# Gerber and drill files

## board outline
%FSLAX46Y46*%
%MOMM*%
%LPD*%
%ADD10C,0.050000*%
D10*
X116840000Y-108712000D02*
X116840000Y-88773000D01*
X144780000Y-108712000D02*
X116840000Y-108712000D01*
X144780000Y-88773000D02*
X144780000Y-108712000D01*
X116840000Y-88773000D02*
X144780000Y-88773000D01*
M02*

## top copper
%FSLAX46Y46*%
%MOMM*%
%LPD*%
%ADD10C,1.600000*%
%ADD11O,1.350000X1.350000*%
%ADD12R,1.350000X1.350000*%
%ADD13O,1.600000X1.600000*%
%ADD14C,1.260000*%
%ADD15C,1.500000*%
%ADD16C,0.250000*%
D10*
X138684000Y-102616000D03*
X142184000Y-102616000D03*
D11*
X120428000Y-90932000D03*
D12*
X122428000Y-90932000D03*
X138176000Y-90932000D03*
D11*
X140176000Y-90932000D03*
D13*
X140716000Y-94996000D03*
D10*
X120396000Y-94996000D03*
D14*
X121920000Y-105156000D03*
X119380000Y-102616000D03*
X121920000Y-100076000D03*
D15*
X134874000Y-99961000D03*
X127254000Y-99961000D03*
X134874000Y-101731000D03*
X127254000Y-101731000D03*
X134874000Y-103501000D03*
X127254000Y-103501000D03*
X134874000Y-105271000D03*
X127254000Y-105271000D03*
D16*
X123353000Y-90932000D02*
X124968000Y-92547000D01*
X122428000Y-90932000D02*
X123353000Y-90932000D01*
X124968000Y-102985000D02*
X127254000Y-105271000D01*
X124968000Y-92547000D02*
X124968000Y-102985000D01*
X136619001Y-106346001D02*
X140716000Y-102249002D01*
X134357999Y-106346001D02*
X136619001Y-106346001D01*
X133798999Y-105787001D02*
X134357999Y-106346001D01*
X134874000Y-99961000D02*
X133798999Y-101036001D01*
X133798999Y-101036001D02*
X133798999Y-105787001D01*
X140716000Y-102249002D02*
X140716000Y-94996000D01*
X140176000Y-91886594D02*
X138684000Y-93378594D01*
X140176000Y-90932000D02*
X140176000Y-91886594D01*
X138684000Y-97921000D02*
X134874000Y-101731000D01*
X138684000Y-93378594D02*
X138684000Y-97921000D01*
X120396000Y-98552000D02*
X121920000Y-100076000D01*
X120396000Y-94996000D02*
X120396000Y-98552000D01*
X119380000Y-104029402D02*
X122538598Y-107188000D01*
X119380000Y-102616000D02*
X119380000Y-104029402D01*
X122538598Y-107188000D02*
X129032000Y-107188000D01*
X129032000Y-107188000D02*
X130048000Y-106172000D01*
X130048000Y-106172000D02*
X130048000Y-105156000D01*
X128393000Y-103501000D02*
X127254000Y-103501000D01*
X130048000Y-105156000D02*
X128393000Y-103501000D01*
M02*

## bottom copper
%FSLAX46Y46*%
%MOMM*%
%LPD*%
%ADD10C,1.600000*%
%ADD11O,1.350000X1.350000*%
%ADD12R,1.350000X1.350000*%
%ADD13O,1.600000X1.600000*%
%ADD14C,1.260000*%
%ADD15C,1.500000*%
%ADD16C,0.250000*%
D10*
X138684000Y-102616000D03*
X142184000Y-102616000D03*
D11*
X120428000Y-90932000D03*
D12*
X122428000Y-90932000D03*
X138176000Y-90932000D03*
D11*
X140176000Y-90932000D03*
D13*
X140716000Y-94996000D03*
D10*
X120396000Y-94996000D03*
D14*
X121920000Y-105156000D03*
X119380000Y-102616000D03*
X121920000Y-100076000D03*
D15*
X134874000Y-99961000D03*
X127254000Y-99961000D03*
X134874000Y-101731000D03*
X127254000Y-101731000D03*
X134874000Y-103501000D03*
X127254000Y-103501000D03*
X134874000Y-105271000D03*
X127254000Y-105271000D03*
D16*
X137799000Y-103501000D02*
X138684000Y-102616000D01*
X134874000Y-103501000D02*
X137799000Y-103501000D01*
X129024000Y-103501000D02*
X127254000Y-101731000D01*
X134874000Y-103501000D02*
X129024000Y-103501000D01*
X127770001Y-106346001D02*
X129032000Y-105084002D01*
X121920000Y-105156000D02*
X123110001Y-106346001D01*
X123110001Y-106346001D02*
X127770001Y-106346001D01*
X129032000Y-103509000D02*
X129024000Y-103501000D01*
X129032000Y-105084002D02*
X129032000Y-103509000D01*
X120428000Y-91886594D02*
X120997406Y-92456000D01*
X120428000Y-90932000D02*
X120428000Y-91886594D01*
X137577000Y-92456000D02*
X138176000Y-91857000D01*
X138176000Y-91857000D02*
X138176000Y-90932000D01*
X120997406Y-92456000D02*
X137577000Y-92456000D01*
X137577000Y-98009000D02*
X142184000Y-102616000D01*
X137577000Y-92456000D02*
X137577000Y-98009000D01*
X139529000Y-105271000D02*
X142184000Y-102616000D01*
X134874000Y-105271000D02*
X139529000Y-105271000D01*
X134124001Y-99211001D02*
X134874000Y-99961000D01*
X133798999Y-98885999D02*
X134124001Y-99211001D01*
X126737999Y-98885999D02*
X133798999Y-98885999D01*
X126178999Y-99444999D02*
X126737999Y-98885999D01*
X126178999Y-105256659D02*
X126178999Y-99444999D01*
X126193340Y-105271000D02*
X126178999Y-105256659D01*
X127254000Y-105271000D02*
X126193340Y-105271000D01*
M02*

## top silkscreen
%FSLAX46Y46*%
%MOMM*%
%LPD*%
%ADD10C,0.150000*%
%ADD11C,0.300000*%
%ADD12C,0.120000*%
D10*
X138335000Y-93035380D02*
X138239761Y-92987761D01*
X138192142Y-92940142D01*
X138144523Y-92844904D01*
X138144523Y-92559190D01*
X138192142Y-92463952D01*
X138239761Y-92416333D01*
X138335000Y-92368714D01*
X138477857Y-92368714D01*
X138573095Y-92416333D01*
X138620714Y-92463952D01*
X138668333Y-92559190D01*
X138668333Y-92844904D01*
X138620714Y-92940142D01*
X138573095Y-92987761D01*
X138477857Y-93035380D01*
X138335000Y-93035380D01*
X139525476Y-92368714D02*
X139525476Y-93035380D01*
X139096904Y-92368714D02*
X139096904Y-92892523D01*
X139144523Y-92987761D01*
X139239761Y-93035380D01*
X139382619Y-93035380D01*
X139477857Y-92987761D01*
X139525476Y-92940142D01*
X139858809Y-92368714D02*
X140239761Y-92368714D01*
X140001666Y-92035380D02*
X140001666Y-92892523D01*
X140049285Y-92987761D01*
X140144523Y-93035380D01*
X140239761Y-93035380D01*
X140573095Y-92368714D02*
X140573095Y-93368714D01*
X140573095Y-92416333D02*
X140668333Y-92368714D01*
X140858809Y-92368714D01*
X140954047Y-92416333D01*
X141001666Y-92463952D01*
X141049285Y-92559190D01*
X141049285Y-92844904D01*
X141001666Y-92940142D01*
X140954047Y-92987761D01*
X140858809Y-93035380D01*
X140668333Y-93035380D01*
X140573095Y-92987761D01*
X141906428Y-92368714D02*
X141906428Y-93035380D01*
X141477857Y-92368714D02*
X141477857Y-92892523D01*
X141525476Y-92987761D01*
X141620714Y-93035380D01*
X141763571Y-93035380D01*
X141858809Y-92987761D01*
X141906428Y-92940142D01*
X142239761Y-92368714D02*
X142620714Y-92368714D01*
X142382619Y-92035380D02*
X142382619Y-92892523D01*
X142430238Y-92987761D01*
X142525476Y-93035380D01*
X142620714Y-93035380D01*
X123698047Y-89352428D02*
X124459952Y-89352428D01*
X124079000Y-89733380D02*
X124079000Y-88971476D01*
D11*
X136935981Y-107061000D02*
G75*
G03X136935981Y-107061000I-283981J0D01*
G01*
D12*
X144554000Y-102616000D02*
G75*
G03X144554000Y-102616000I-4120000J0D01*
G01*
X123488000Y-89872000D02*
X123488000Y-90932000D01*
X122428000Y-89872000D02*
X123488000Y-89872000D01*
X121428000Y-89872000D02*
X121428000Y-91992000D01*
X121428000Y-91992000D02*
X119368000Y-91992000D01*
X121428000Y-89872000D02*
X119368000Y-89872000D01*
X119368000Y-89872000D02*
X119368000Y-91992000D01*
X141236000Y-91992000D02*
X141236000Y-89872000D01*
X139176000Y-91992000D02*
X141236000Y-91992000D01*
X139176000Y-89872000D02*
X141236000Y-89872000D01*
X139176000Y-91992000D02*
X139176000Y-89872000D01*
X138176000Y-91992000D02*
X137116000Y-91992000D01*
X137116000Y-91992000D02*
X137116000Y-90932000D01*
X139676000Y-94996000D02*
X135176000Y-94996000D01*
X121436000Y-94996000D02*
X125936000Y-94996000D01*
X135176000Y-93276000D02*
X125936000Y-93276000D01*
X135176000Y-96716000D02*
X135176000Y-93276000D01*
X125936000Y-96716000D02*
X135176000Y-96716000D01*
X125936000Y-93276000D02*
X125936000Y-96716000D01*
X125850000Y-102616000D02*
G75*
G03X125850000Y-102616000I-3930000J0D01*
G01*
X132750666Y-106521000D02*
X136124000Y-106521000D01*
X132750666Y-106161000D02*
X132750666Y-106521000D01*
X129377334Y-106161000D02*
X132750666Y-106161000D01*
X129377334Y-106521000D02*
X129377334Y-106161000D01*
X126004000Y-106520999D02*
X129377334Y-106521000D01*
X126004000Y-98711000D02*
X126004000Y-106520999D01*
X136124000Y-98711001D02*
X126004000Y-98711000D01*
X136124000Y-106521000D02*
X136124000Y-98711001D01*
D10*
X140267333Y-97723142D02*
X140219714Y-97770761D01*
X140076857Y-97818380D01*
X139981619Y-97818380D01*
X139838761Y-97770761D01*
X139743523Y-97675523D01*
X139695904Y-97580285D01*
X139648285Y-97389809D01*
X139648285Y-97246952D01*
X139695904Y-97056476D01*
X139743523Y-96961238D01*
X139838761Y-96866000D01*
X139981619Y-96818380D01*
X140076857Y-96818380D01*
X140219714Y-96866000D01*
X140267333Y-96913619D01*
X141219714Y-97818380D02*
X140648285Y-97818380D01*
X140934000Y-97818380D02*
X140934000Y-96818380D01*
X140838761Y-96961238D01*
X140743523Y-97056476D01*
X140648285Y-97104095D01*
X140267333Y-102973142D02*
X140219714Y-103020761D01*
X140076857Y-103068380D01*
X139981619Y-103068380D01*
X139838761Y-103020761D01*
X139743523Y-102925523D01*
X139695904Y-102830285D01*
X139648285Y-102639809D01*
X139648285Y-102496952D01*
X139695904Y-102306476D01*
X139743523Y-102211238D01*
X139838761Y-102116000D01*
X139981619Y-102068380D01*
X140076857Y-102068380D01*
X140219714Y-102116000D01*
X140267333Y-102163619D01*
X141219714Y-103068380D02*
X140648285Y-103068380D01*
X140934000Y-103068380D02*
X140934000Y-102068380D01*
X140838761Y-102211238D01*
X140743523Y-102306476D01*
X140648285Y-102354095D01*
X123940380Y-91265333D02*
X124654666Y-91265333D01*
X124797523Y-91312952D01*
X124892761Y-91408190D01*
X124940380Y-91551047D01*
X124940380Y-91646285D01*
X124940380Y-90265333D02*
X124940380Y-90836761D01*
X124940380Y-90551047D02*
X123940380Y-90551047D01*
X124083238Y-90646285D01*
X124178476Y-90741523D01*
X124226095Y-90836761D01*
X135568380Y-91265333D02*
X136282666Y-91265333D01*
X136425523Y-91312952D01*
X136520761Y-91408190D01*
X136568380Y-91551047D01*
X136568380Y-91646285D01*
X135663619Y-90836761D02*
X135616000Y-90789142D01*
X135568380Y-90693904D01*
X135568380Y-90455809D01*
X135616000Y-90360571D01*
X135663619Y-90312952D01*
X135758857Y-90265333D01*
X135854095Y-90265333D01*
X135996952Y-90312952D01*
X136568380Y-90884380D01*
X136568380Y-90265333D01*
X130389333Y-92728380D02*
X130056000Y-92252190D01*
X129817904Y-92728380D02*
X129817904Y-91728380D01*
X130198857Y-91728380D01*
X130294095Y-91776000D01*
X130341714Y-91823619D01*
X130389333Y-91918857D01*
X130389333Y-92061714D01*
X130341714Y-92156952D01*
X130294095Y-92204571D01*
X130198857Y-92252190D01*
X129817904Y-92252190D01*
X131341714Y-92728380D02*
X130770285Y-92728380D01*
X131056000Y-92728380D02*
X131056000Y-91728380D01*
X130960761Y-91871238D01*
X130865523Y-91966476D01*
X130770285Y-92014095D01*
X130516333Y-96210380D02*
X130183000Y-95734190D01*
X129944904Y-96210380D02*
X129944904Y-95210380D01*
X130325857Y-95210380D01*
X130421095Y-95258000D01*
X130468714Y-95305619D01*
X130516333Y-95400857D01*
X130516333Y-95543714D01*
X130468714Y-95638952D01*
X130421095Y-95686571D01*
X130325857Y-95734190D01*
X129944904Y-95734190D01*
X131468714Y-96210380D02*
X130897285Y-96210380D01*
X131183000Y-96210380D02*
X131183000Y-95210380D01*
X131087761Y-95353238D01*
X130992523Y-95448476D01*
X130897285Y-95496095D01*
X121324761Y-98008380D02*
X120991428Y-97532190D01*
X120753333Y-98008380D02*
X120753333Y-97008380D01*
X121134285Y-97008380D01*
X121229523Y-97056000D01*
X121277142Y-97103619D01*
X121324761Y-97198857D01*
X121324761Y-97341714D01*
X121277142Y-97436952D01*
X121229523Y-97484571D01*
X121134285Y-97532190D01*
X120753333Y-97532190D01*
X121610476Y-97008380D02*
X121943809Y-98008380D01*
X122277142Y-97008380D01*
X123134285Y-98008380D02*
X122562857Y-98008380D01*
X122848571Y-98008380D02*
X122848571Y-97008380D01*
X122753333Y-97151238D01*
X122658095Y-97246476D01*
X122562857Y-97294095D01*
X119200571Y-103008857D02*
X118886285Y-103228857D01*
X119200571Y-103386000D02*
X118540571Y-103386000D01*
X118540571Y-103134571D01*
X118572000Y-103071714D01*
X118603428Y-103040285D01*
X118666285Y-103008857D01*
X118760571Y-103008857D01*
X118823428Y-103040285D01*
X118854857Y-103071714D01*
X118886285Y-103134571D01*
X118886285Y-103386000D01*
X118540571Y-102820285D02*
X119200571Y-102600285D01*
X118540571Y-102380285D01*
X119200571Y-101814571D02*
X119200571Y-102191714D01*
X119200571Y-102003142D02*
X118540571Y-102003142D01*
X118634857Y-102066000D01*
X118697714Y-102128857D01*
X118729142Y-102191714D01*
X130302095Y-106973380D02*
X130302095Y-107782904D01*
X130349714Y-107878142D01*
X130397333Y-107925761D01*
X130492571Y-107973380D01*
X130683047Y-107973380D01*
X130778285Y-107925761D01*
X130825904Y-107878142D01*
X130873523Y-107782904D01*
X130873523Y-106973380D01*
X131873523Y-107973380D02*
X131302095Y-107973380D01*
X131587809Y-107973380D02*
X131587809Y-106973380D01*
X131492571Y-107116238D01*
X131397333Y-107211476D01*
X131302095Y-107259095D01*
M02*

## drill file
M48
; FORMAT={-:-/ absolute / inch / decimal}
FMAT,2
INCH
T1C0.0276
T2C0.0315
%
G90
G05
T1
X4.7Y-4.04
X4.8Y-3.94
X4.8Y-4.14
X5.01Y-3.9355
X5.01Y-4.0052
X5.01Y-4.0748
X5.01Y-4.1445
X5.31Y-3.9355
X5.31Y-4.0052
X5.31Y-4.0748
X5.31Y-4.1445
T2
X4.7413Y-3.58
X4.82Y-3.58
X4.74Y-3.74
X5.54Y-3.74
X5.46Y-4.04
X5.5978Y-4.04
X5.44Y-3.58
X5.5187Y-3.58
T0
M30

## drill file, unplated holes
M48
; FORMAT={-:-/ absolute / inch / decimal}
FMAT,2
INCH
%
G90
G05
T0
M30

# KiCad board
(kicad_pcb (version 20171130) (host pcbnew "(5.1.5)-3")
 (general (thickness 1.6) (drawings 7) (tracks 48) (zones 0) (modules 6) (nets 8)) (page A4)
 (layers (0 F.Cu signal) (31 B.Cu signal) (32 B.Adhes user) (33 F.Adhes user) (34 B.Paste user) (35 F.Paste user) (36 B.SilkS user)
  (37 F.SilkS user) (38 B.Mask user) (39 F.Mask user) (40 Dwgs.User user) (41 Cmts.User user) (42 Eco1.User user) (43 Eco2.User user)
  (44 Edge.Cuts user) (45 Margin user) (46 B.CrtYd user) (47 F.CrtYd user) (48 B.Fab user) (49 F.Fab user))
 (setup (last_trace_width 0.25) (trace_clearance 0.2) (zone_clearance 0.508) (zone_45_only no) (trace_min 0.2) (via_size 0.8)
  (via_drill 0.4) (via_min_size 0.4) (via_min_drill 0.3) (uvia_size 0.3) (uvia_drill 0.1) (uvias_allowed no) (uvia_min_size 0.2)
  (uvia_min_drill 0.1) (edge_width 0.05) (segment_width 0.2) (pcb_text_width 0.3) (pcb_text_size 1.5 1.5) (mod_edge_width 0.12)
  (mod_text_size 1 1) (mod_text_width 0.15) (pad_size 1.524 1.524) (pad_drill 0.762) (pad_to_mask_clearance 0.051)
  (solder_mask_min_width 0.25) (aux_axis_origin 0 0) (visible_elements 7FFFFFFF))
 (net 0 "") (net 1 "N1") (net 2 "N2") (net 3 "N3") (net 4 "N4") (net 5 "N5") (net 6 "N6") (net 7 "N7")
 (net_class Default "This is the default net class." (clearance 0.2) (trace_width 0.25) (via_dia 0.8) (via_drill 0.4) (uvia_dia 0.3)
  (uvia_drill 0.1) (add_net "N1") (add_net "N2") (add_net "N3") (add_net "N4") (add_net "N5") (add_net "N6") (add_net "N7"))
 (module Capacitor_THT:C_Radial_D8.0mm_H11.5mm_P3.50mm (layer F.Cu) (at 138.684 102.616)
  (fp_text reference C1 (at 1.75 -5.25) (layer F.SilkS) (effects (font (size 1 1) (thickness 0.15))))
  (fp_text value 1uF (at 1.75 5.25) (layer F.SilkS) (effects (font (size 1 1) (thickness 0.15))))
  (fp_circle (center 1.75 0) (end 5.87 0) (layer F.SilkS) (width 0.12))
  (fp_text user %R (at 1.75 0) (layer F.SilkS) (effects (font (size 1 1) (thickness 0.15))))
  (pad 1 thru_hole circle (at 0 0) (size 1.6 1.6) (drill 0.8) (layers *.Cu *.Mask) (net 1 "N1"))
  (pad 2 thru_hole circle (at 3.5 0) (size 1.6 1.6) (drill 0.8) (layers *.Cu *.Mask) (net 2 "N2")))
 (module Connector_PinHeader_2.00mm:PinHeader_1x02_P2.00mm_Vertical (layer F.Cu) (at 122.428 90.932 270)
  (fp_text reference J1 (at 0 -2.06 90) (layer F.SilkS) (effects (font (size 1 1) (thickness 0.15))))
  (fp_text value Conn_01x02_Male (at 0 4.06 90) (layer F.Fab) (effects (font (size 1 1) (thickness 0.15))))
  (fp_line (start -1.06 -1.06) (end 0 -1.06) (layer F.SilkS) (width 0.12))
  (fp_line (start -1.06 0) (end -1.06 -1.06) (layer F.SilkS) (width 0.12))
  (fp_line (start -1.06 1) (end 1.06 1) (layer F.SilkS) (width 0.12))
  (fp_line (start 1.06 1) (end 1.06 3.06) (layer F.SilkS) (width 0.12))
  (fp_line (start -1.06 1) (end -1.06 3.06) (layer F.SilkS) (width 0.12))
  (fp_line (start -1.06 3.06) (end 1.06 3.06) (layer F.SilkS) (width 0.12))
  (pad 2 thru_hole oval (at 0 2 270) (size 1.35 1.35) (drill 0.8) (layers *.Cu *.Mask) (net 2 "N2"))
  (pad 1 thru_hole rect (at 0 0 270) (size 1.35 1.35) (drill 0.8) (layers *.Cu *.Mask) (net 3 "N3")))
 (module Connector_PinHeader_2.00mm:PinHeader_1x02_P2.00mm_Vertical (layer F.Cu) (at 138.176 90.932 90)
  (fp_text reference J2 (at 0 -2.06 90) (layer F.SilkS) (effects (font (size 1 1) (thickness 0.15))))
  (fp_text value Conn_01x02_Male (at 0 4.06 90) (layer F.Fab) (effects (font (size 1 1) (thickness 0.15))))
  (fp_line (start -1.06 3.06) (end 1.06 3.06) (layer F.SilkS) (width 0.12))
  (fp_line (start -1.06 1) (end -1.06 3.06) (layer F.SilkS) (width 0.12))
  (fp_line (start 1.06 1) (end 1.06 3.06) (layer F.SilkS) (width 0.12))
  (fp_line (start -1.06 1) (end 1.06 1) (layer F.SilkS) (width 0.12))
  (fp_line (start -1.06 0) (end -1.06 -1.06) (layer F.SilkS) (width 0.12))
  (fp_line (start -1.06 -1.06) (end 0 -1.06) (layer F.SilkS) (width 0.12))
  (pad 1 thru_hole rect (at 0 0 90) (size 1.35 1.35) (drill 0.8) (layers *.Cu *.Mask) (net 2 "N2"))
  (pad 2 thru_hole oval (at 0 2 90) (size 1.35 1.35) (drill 0.8) (layers *.Cu *.Mask) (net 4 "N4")))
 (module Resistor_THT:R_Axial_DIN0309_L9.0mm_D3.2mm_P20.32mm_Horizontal (layer F.Cu) (at 120.396 94.996)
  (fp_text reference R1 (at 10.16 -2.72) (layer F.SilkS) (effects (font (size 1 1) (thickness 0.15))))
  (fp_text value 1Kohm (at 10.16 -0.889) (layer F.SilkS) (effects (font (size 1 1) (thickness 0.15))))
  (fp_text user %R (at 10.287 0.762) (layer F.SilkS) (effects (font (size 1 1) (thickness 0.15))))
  (fp_line (start 19.28 0) (end 14.78 0) (layer F.SilkS) (width 0.12))
  (fp_line (start 1.04 0) (end 5.54 0) (layer F.SilkS) (width 0.12))
  (fp_line (start 14.78 -1.72) (end 5.54 -1.72) (layer F.SilkS) (width 0.12))
  (fp_line (start 14.78 1.72) (end 14.78 -1.72) (layer F.SilkS) (width 0.12))
  (fp_line (start 5.54 1.72) (end 14.78 1.72) (layer F.SilkS) (width 0.12))
  (fp_line (start 5.54 -1.72) (end 5.54 1.72) (layer F.SilkS) (width 0.12))
  (pad 2 thru_hole oval (at 20.32 0) (size 1.6 1.6) (drill 0.8) (layers *.Cu *.Mask) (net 3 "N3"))
  (pad 1 thru_hole circle (at 0 0) (size 1.6 1.6) (drill 0.8) (layers *.Cu *.Mask) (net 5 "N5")))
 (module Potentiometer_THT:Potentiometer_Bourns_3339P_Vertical (layer F.Cu) (at 121.92 105.156)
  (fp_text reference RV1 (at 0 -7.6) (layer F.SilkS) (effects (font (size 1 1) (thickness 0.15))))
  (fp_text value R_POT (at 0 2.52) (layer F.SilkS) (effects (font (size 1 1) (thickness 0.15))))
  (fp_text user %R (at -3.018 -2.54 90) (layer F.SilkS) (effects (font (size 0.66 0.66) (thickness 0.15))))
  (fp_circle (center 0 -2.54) (end 3.93 -2.54) (layer F.SilkS) (width 0.12))
  (pad 1 thru_hole circle (at 0 0) (size 1.26 1.26) (drill 0.7) (layers *.Cu *.Mask) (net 1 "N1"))
  (pad 2 thru_hole circle (at -2.54 -2.54) (size 1.26 1.26) (drill 0.7) (layers *.Cu *.Mask) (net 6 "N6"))
  (pad 3 thru_hole circle (at 0 -5.08) (size 1.26 1.26) (drill 0.7) (layers *.Cu *.Mask) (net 5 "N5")))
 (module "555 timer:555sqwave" (layer F.Cu) (at 131.064 102.616 90)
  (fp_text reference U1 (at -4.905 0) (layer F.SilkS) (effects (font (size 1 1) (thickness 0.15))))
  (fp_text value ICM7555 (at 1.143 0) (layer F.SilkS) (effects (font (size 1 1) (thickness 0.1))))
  (fp_line (start -3.905 1.686666) (end -3.905 5.06) (layer F.SilkS) (width 0.12))
  (fp_line (start -3.545 1.686666) (end -3.905 1.686666) (layer F.SilkS) (width 0.12))
  (fp_line (start -3.545 -1.686666) (end -3.545 1.686666) (layer F.SilkS) (width 0.12))
  (fp_line (start -3.905 -1.686666) (end -3.545 -1.686666) (layer F.SilkS) (width 0.12))
  (fp_line (start -3.904999 -5.06) (end -3.905 -1.686666) (layer F.SilkS) (width 0.12))
  (fp_line (start 3.905 -5.06) (end -3.904999 -5.06) (layer F.SilkS) (width 0.12))
  (fp_line (start 3.904999 5.06) (end 3.905 -5.06) (layer F.SilkS) (width 0.12))
  (fp_line (start -3.905 5.06) (end 3.904999 5.06) (layer F.SilkS) (width 0.12))
  (pad 4 thru_hole circle (at 2.655 3.81 90) (size 1.5 1.5) (drill 0.7) (layers *.Cu *.Mask) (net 3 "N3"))
  (pad 5 thru_hole circle (at 2.655 -3.81 90) (size 1.5 1.5) (drill 0.7) (layers *.Cu *.Mask) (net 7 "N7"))
  (pad 3 thru_hole circle (at 0.885 3.81 90) (size 1.5 1.5) (drill 0.7) (layers *.Cu *.Mask) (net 4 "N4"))
  (pad 6 thru_hole circle (at 0.885 -3.81 90) (size 1.5 1.5) (drill 0.7) (layers *.Cu *.Mask) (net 1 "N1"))
  (pad 2 thru_hole circle (at -0.885 3.81 90) (size 1.5 1.5) (drill 0.7) (layers *.Cu *.Mask) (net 1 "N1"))
  (pad 7 thru_hole circle (at -0.885 -3.81 90) (size 1.5 1.5) (drill 0.7) (layers *.Cu *.Mask) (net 6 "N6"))
  (pad 1 thru_hole circle (at -2.655 3.81 90) (size 1.5 1.5) (drill 0.7) (layers *.Cu *.Mask) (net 2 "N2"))
  (pad 8 thru_hole circle (at -2.655 -3.81 90) (size 1.5 1.5) (drill 0.7) (layers *.Cu *.Mask) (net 3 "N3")))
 (gr_line (start 116.84 108.712) (end 116.84 88.773) (layer Edge.Cuts) (width 0.05))
 (gr_line (start 144.78 108.712) (end 116.84 108.712) (layer Edge.Cuts) (width 0.05))
 (gr_line (start 144.78 88.773) (end 144.78 108.712) (layer Edge.Cuts) (width 0.05))
 (gr_line (start 116.84 88.773) (end 144.78 88.773) (layer Edge.Cuts) (width 0.05))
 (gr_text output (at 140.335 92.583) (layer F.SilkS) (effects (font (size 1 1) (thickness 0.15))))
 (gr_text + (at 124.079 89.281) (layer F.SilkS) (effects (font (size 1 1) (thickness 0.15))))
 (gr_circle (center 136.652 107.061) (end 136.935981 107.061) (layer F.SilkS) (width 0.3))
 (segment (start 137.799 103.501) (end 138.684 102.616) (width 0.25) (layer B.Cu) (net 1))
 (segment (start 134.874 103.501) (end 137.799 103.501) (width 0.25) (layer B.Cu) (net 1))
 (segment (start 129.024 103.501) (end 127.254 101.731) (width 0.25) (layer B.Cu) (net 1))
 (segment (start 134.874 103.501) (end 129.024 103.501) (width 0.25) (layer B.Cu) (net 1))
 (segment (start 127.770001 106.346001) (end 129.032 105.084002) (width 0.25) (layer B.Cu) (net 1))
 (segment (start 121.92 105.156) (end 123.110001 106.346001) (width 0.25) (layer B.Cu) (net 1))
 (segment (start 123.110001 106.346001) (end 127.770001 106.346001) (width 0.25) (layer B.Cu) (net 1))
 (segment (start 129.032 103.509) (end 129.024 103.501) (width 0.25) (layer B.Cu) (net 1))
 (segment (start 129.032 105.084002) (end 129.032 103.509) (width 0.25) (layer B.Cu) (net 1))
 (segment (start 120.428 91.886594) (end 120.997406 92.456) (width 0.25) (layer B.Cu) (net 2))
 (segment (start 120.428 90.932) (end 120.428 91.886594) (width 0.25) (layer B.Cu) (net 2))
 (segment (start 137.577 92.456) (end 138.176 91.857) (width 0.25) (layer B.Cu) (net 2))
 (segment (start 138.176 91.857) (end 138.176 90.932) (width 0.25) (layer B.Cu) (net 2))
 (segment (start 120.997406 92.456) (end 137.577 92.456) (width 0.25) (layer B.Cu) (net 2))
 (segment (start 137.577 98.009) (end 142.184 102.616) (width 0.25) (layer B.Cu) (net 2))
 (segment (start 137.577 92.456) (end 137.577 98.009) (width 0.25) (layer B.Cu) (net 2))
 (segment (start 139.529 105.271) (end 142.184 102.616) (width 0.25) (layer B.Cu) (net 2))
 (segment (start 134.874 105.271) (end 139.529 105.271) (width 0.25) (layer B.Cu) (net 2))
 (segment (start 123.353 90.932) (end 124.968 92.547) (width 0.25) (layer F.Cu) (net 3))
 (segment (start 122.428 90.932) (end 123.353 90.932) (width 0.25) (layer F.Cu) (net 3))
 (segment (start 124.968 102.985) (end 127.254 105.271) (width 0.25) (layer F.Cu) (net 3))
 (segment (start 124.968 92.547) (end 124.968 102.985) (width 0.25) (layer F.Cu) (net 3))
 (segment (start 134.124001 99.211001) (end 134.874 99.961) (width 0.25) (layer B.Cu) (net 3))
 (segment (start 133.798999 98.885999) (end 134.124001 99.211001) (width 0.25) (layer B.Cu) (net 3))
 (segment (start 126.737999 98.885999) (end 133.798999 98.885999) (width 0.25) (layer B.Cu) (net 3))
 (segment (start 126.178999 99.444999) (end 126.737999 98.885999) (width 0.25) (layer B.Cu) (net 3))
 (segment (start 126.178999 105.256659) (end 126.178999 99.444999) (width 0.25) (layer B.Cu) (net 3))
 (segment (start 126.19334 105.271) (end 126.178999 105.256659) (width 0.25) (layer B.Cu) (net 3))
 (segment (start 127.254 105.271) (end 126.19334 105.271) (width 0.25) (layer B.Cu) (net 3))
 (segment (start 136.619001 106.346001) (end 140.716 102.249002) (width 0.25) (layer F.Cu) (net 3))
 (segment (start 134.357999 106.346001) (end 136.619001 106.346001) (width 0.25) (layer F.Cu) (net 3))
 (segment (start 133.798999 105.787001) (end 134.357999 106.346001) (width 0.25) (layer F.Cu) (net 3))
 (segment (start 134.874 99.961) (end 133.798999 101.036001) (width 0.25) (layer F.Cu) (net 3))
 (segment (start 133.798999 101.036001) (end 133.798999 105.787001) (width 0.25) (layer F.Cu) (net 3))
 (segment (start 140.716 102.249002) (end 140.716 94.996) (width 0.25) (layer F.Cu) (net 3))
 (segment (start 140.176 91.886594) (end 138.684 93.378594) (width 0.25) (layer F.Cu) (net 4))
 (segment (start 140.176 90.932) (end 140.176 91.886594) (width 0.25) (layer F.Cu) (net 4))
 (segment (start 138.684 97.921) (end 134.874 101.731) (width 0.25) (layer F.Cu) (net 4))
 (segment (start 138.684 93.378594) (end 138.684 97.921) (width 0.25) (layer F.Cu) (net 4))
 (segment (start 120.396 98.552) (end 121.92 100.076) (width 0.25) (layer F.Cu) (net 5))
 (segment (start 120.396 94.996) (end 120.396 98.552) (width 0.25) (layer F.Cu) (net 5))
 (segment (start 119.38 104.029402) (end 122.538598 107.188) (width 0.25) (layer F.Cu) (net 6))
 (segment (start 119.38 102.616) (end 119.38 104.029402) (width 0.25) (layer F.Cu) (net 6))
 (segment (start 122.538598 107.188) (end 129.032 107.188) (width 0.25) (layer F.Cu) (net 6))
 (segment (start 129.032 107.188) (end 130.048 106.172) (width 0.25) (layer F.Cu) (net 6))
 (segment (start 130.048 106.172) (end 130.048 105.156) (width 0.25) (layer F.Cu) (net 6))
 (segment (start 128.393 103.501) (end 127.254 103.501) (width 0.25) (layer F.Cu) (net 6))
 (segment (start 130.048 105.156) (end 128.393 103.501) (width 0.25) (layer F.Cu) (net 6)))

